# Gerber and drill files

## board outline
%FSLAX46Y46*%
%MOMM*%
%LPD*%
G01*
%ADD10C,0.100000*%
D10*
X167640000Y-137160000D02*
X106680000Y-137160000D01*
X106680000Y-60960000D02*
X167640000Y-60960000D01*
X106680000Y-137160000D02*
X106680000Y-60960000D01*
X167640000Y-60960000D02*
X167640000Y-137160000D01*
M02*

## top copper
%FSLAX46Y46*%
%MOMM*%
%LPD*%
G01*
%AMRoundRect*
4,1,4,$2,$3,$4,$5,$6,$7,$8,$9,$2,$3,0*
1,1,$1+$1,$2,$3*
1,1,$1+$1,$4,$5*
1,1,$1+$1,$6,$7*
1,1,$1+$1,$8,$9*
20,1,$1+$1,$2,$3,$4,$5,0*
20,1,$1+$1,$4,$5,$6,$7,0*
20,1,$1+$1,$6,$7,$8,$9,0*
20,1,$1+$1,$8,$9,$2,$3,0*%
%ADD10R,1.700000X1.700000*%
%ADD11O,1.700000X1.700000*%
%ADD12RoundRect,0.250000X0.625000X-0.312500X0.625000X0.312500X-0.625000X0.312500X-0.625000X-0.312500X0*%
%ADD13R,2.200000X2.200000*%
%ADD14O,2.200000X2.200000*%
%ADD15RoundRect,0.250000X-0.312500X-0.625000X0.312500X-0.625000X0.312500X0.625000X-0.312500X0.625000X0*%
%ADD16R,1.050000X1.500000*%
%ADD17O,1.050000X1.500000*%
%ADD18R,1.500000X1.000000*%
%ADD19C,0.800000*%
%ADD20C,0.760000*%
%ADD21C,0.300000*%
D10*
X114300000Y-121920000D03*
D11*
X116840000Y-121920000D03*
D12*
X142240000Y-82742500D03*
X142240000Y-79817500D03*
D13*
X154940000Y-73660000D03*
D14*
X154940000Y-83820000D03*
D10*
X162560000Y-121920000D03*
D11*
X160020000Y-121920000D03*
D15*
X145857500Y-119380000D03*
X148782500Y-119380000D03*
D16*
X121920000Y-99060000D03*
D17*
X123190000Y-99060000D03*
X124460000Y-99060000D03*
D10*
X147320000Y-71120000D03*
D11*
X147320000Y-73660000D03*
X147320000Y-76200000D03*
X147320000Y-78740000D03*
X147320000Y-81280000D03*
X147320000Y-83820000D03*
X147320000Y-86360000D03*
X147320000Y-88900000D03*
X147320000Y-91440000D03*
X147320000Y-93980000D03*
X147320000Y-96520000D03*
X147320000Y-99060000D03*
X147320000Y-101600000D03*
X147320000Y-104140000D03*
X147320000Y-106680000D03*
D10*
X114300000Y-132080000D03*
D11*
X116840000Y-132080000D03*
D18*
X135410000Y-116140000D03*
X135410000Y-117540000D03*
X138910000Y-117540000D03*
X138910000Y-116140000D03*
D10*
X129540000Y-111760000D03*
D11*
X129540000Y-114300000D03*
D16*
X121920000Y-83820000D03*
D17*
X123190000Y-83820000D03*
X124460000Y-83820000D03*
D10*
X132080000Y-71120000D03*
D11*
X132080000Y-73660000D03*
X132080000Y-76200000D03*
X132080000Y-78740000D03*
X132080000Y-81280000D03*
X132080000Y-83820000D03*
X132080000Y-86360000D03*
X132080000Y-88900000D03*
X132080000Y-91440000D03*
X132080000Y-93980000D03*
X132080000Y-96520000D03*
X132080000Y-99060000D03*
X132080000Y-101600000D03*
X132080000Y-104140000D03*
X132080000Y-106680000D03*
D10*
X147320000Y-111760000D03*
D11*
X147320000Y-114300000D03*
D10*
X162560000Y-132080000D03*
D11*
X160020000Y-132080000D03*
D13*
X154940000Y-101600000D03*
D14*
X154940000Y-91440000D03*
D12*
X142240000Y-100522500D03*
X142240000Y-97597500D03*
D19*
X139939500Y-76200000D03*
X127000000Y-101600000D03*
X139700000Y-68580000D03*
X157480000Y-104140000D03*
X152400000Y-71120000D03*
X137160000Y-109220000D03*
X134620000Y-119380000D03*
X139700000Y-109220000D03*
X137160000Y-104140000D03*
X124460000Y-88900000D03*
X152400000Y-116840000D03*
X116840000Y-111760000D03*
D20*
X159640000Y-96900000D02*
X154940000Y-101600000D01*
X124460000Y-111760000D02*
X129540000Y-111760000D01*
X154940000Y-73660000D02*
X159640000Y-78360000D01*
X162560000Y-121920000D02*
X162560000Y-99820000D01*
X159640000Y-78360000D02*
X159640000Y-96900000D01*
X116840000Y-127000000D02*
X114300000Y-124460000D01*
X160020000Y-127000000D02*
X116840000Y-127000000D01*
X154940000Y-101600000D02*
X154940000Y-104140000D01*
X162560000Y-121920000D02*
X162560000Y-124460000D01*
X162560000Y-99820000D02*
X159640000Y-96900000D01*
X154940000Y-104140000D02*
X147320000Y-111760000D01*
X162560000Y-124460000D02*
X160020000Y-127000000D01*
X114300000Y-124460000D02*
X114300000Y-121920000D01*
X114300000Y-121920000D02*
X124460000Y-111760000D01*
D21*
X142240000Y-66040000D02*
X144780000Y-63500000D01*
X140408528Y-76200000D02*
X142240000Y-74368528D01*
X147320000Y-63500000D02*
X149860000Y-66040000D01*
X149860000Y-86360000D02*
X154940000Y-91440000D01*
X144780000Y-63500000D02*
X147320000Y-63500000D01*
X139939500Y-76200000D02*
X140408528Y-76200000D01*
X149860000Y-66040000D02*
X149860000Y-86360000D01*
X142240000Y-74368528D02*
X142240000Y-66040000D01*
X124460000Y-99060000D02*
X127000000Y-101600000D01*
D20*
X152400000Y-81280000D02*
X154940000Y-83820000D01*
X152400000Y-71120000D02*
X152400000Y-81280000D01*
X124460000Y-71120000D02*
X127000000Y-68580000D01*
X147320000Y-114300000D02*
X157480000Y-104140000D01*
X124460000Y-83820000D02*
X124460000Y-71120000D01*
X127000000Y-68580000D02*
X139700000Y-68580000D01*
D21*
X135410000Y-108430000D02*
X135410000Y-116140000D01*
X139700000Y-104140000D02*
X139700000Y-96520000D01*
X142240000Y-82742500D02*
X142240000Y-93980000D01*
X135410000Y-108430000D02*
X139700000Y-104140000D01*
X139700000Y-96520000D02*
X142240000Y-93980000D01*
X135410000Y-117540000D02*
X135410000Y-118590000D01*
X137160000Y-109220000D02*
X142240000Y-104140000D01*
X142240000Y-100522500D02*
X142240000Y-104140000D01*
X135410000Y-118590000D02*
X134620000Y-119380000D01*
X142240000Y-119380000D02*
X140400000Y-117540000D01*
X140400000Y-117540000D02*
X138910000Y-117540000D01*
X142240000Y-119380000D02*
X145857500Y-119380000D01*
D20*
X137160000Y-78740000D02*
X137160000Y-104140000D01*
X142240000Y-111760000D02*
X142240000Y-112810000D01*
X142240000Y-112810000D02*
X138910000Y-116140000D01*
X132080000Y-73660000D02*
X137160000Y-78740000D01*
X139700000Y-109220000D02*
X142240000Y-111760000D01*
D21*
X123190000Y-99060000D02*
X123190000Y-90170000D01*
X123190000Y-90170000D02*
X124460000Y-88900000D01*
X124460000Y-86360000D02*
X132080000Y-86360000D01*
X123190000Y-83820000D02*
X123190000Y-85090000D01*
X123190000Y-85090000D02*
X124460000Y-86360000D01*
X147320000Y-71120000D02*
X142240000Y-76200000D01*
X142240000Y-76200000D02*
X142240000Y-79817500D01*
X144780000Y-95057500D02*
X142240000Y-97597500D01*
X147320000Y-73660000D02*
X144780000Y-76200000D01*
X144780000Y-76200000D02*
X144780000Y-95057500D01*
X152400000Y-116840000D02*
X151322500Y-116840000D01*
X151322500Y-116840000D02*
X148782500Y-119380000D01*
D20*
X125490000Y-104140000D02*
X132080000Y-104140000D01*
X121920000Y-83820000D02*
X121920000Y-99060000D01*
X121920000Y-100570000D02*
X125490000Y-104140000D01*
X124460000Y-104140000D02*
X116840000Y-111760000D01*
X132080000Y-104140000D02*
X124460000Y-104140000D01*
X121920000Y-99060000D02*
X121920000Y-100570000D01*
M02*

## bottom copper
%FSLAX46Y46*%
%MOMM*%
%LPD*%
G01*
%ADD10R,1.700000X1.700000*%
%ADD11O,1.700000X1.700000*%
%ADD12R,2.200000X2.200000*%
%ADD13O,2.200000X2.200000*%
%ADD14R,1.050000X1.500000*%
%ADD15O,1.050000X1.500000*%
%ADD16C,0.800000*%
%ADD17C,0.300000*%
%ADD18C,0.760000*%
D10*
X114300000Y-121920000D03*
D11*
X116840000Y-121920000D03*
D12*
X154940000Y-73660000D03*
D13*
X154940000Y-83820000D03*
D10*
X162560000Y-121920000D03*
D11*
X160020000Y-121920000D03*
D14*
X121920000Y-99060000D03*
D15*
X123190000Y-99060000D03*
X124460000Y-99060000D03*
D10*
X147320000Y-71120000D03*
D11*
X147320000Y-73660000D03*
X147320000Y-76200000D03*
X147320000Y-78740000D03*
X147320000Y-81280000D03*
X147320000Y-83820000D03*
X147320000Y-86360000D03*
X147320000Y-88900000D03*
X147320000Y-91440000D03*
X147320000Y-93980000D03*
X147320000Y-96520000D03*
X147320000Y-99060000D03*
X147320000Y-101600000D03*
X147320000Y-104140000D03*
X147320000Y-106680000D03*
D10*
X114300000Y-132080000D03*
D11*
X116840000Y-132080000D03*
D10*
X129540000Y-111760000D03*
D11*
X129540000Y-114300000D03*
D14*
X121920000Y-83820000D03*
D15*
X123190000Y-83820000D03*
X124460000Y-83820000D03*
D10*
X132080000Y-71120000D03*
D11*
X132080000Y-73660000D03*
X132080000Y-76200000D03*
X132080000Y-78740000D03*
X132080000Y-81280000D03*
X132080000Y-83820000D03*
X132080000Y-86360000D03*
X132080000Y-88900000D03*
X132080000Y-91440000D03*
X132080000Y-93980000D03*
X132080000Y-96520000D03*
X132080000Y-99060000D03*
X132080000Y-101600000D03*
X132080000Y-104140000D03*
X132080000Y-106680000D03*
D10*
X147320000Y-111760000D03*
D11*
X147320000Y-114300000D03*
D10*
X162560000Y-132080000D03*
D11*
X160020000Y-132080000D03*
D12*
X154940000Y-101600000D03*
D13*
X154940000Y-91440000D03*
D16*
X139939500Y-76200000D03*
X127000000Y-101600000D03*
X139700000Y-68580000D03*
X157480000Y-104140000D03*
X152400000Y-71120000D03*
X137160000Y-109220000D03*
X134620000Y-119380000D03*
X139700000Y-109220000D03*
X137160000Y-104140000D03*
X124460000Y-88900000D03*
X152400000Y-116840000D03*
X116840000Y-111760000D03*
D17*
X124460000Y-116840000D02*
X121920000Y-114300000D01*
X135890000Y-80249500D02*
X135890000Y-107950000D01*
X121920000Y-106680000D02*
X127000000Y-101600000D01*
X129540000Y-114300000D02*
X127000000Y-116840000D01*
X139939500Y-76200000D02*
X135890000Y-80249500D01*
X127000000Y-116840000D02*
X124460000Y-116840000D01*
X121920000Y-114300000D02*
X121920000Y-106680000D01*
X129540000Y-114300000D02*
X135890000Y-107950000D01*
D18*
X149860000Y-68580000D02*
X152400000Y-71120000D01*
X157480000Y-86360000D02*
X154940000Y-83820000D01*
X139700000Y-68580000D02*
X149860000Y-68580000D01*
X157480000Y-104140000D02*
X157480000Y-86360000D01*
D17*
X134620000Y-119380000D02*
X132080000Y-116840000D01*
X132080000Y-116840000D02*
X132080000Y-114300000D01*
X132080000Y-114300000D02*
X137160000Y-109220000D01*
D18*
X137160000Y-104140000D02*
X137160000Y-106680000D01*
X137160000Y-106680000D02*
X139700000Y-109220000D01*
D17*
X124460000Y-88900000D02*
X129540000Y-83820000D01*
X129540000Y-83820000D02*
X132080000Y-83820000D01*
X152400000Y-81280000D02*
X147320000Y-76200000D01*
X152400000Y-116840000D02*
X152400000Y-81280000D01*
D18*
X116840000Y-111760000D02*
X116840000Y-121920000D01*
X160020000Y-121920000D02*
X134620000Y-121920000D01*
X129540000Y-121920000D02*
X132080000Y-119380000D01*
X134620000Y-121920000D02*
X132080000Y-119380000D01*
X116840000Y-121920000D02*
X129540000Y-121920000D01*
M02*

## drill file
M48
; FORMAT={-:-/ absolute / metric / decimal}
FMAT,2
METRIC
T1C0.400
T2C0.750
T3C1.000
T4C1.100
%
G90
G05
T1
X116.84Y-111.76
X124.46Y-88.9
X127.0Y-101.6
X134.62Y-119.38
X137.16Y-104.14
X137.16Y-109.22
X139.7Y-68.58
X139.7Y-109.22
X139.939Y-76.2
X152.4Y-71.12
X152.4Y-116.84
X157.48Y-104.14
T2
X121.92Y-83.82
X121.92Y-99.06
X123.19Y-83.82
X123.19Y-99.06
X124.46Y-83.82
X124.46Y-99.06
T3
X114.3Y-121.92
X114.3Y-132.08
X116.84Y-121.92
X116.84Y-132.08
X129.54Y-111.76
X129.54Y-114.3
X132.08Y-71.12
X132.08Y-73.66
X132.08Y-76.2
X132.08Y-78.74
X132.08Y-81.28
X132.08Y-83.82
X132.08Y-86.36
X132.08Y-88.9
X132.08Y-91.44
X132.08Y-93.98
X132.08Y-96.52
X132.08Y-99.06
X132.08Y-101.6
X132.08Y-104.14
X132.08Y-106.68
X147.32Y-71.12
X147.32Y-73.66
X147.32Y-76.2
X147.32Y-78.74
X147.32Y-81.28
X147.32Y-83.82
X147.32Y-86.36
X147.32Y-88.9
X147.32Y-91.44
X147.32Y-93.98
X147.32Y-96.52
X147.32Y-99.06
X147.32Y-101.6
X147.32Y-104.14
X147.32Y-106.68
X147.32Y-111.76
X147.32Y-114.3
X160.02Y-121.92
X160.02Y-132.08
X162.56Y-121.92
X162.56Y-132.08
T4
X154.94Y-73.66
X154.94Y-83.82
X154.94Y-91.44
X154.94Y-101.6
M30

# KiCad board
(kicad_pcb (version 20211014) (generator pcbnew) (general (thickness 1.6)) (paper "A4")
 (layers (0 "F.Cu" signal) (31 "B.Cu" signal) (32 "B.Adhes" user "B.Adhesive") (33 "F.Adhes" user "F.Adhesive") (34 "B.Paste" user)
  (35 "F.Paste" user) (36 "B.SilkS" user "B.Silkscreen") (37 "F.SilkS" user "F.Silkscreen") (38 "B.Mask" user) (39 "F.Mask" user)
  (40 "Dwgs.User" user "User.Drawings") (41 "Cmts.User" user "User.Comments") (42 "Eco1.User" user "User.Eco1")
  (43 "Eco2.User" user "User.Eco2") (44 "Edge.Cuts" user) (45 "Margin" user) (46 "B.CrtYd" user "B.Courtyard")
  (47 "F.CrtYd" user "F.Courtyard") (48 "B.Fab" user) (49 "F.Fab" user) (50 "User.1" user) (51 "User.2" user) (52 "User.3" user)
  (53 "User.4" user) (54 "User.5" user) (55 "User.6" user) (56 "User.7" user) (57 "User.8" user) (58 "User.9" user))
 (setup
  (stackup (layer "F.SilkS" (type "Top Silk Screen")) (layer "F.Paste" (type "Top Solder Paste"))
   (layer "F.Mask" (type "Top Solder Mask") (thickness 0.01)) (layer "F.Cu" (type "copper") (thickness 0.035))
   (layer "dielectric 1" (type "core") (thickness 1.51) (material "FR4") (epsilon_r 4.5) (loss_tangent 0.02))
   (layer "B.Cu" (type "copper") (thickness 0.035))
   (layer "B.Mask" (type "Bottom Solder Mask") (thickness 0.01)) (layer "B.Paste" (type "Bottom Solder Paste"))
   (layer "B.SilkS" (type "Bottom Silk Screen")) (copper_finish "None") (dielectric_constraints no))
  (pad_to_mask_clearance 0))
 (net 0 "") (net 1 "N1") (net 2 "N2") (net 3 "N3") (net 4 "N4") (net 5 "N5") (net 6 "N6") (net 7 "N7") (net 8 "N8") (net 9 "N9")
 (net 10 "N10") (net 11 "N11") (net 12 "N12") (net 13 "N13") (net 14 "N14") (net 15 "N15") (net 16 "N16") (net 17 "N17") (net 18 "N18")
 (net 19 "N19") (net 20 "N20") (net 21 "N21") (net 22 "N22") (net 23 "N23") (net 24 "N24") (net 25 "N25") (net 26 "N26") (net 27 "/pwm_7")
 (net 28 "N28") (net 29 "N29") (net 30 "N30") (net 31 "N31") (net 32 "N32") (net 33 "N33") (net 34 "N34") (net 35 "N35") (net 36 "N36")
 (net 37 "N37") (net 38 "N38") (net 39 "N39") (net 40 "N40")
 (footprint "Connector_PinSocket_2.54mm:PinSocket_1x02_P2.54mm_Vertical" (layer "F.Cu") (at 114.3 121.92 90)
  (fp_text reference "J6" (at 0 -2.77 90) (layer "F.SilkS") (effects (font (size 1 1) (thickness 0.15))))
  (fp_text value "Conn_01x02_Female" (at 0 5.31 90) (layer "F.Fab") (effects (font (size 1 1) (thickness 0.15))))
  (pad "1" thru_hole rect (at 0 0 90) (size 1.7 1.7) (drill 1) (layers *.Cu *.Mask) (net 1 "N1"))
  (pad "2" thru_hole oval (at 0 2.54 90) (size 1.7 1.7) (drill 1) (layers *.Cu *.Mask) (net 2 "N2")))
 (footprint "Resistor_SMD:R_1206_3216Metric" (layer "F.Cu") (at 142.24 81.28 90)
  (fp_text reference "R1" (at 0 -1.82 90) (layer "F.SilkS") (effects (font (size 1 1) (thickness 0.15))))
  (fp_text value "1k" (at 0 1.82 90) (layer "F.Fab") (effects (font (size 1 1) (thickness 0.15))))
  (pad "1" smd roundrect (at -1.4625 0 90) (size 1.125 1.75) (layers "F.Cu" "F.Paste" "F.Mask") (roundrect_rratio 0.222222) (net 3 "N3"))
  (pad "2" smd roundrect (at 1.4625 0 90) (size 1.125 1.75) (layers "F.Cu" "F.Paste" "F.Mask") (roundrect_rratio 0.222222) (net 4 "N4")))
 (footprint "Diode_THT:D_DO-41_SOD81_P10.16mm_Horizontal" (layer "F.Cu") (at 154.94 73.66 -90)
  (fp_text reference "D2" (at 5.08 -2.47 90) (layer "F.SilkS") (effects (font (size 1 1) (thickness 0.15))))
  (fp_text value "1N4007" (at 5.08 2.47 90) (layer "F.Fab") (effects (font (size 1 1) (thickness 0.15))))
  (pad "1" thru_hole rect (at 0 0 270) (size 2.2 2.2) (drill 1.1) (layers *.Cu *.Mask) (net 1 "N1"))
  (pad "2" thru_hole oval (at 10.16 0 270) (size 2.2 2.2) (drill 1.1) (layers *.Cu *.Mask) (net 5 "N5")))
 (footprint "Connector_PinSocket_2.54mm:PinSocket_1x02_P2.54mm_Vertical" (layer "F.Cu") (at 162.56 121.92 -90)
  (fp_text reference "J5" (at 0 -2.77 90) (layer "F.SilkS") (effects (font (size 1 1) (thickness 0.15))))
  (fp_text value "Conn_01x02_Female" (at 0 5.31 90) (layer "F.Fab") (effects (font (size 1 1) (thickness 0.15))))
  (pad "1" thru_hole rect (at 0 0 270) (size 1.7 1.7) (drill 1) (layers *.Cu *.Mask) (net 1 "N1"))
  (pad "2" thru_hole oval (at 0 2.54 270) (size 1.7 1.7) (drill 1) (layers *.Cu *.Mask) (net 2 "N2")))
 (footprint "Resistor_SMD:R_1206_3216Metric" (layer "F.Cu") (at 147.32 119.38)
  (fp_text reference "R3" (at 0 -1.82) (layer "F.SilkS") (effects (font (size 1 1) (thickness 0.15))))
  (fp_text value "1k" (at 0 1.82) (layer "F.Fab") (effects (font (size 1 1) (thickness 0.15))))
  (pad "1" smd roundrect (at -1.4625 0) (size 1.125 1.75) (layers "F.Cu" "F.Paste" "F.Mask") (roundrect_rratio 0.222222) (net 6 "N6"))
  (pad "2" smd roundrect (at 1.4625 0) (size 1.125 1.75) (layers "F.Cu" "F.Paste" "F.Mask") (roundrect_rratio 0.222222) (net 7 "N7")))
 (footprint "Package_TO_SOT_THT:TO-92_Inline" (layer "F.Cu") (at 121.92 99.06)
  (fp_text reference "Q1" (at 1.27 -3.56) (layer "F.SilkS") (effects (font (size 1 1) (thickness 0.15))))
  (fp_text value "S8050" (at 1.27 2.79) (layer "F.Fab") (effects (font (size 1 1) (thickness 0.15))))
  (pad "1" thru_hole rect (at 0 0) (size 1.05 1.5) (drill 0.75) (layers *.Cu *.Mask) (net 2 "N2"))
  (pad "2" thru_hole oval (at 1.27 0) (size 1.05 1.5) (drill 0.75) (layers *.Cu *.Mask) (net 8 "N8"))
  (pad "3" thru_hole oval (at 2.54 0) (size 1.05 1.5) (drill 0.75) (layers *.Cu *.Mask) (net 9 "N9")))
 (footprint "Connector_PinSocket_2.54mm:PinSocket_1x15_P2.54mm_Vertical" (layer "F.Cu") (at 147.32 71.12)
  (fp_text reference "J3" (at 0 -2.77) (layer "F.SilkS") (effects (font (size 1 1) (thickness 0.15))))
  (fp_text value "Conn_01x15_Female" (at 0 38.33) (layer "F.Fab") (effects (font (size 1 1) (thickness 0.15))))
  (pad "1" thru_hole rect (at 0 0) (size 1.7 1.7) (drill 1) (layers *.Cu *.Mask) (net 4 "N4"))
  (pad "2" thru_hole oval (at 0 2.54) (size 1.7 1.7) (drill 1) (layers *.Cu *.Mask) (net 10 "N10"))
  (pad "3" thru_hole oval (at 0 5.08) (size 1.7 1.7) (drill 1) (layers *.Cu *.Mask) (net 7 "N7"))
  (pad "4" thru_hole oval (at 0 7.62) (size 1.7 1.7) (drill 1) (layers *.Cu *.Mask) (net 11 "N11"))
  (pad "5" thru_hole oval (at 0 10.16) (size 1.7 1.7) (drill 1) (layers *.Cu *.Mask) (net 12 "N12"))
  (pad "6" thru_hole oval (at 0 12.7) (size 1.7 1.7) (drill 1) (layers *.Cu *.Mask) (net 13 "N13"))
  (pad "7" thru_hole oval (at 0 15.24) (size 1.7 1.7) (drill 1) (layers *.Cu *.Mask) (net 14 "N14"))
  (pad "8" thru_hole oval (at 0 17.78) (size 1.7 1.7) (drill 1) (layers *.Cu *.Mask) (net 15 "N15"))
  (pad "9" thru_hole oval (at 0 20.32) (size 1.7 1.7) (drill 1) (layers *.Cu *.Mask) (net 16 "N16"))
  (pad "10" thru_hole oval (at 0 22.86) (size 1.7 1.7) (drill 1) (layers *.Cu *.Mask) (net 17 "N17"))
  (pad "11" thru_hole oval (at 0 25.4) (size 1.7 1.7) (drill 1) (layers *.Cu *.Mask) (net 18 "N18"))
  (pad "12" thru_hole oval (at 0 27.94) (size 1.7 1.7) (drill 1) (layers *.Cu *.Mask) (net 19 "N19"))
  (pad "13" thru_hole oval (at 0 30.48) (size 1.7 1.7) (drill 1) (layers *.Cu *.Mask) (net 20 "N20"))
  (pad "14" thru_hole oval (at 0 33.02) (size 1.7 1.7) (drill 1) (layers *.Cu *.Mask) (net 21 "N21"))
  (pad "15" thru_hole oval (at 0 35.56) (size 1.7 1.7) (drill 1) (layers *.Cu *.Mask) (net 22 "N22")))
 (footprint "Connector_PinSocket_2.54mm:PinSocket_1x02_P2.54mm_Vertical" (layer "F.Cu") (at 114.3 132.08 90)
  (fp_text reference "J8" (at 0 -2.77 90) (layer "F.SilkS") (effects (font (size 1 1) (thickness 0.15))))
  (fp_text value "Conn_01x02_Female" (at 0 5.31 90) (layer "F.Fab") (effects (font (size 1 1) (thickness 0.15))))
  (pad "1" thru_hole rect (at 0 0 90) (size 1.7 1.7) (drill 1) (layers *.Cu *.Mask) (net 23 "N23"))
  (pad "2" thru_hole oval (at 0 2.54 90) (size 1.7 1.7) (drill 1) (layers *.Cu *.Mask) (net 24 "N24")))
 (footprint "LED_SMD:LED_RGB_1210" (layer "F.Cu") (at 137.16 116.84)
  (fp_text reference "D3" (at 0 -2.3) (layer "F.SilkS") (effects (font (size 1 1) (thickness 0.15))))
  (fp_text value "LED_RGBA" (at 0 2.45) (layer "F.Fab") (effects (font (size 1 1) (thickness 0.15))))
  (pad "1" smd rect (at -1.75 -0.7 180) (size 1.5 1) (layers "F.Cu" "F.Paste" "F.Mask") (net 3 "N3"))
  (pad "2" smd rect (at -1.75 0.7 180) (size 1.5 1) (layers "F.Cu" "F.Paste" "F.Mask") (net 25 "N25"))
  (pad "3" smd rect (at 1.75 0.7 180) (size 1.5 1) (layers "F.Cu" "F.Paste" "F.Mask") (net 6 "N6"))
  (pad "4" smd rect (at 1.75 -0.7 180) (size 1.5 1) (layers "F.Cu" "F.Paste" "F.Mask") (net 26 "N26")))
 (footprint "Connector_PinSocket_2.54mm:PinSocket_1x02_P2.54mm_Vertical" (layer "F.Cu") (at 129.54 111.76)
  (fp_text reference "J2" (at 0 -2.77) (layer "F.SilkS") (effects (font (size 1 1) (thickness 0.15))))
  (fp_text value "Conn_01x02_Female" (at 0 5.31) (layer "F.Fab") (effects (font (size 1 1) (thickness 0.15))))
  (pad "1" thru_hole rect (at 0 0) (size 1.7 1.7) (drill 1) (layers *.Cu *.Mask) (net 1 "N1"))
  (pad "2" thru_hole oval (at 0 2.54) (size 1.7 1.7) (drill 1) (layers *.Cu *.Mask) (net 9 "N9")))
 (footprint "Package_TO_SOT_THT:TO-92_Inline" (layer "F.Cu") (at 121.92 83.82)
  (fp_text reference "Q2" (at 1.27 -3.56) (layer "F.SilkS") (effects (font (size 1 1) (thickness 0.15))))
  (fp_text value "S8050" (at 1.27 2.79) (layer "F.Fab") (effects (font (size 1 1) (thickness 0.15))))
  (pad "1" thru_hole rect (at 0 0) (size 1.05 1.5) (drill 0.75) (layers *.Cu *.Mask) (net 2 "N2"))
  (pad "2" thru_hole oval (at 1.27 0) (size 1.05 1.5) (drill 0.75) (layers *.Cu *.Mask) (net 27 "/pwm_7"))
  (pad "3" thru_hole oval (at 2.54 0) (size 1.05 1.5) (drill 0.75) (layers *.Cu *.Mask) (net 5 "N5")))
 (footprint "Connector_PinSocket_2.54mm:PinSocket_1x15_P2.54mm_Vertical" (layer "F.Cu") (at 132.08 71.12)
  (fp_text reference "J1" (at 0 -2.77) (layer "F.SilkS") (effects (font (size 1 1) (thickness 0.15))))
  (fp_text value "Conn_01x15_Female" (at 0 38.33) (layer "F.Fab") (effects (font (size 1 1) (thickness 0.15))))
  (pad "1" thru_hole rect (at 0 0) (size 1.7 1.7) (drill 1) (layers *.Cu *.Mask) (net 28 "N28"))
  (pad "2" thru_hole oval (at 0 2.54) (size 1.7 1.7) (drill 1) (layers *.Cu *.Mask) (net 26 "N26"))
  (pad "3" thru_hole oval (at 0 5.08) (size 1.7 1.7) (drill 1) (layers *.Cu *.Mask) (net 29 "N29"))
  (pad "4" thru_hole oval (at 0 7.62) (size 1.7 1.7) (drill 1) (layers *.Cu *.Mask) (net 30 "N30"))
  (pad "5" thru_hole oval (at 0 10.16) (size 1.7 1.7) (drill 1) (layers *.Cu *.Mask) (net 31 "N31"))
  (pad "6" thru_hole oval (at 0 12.7) (size 1.7 1.7) (drill 1) (layers *.Cu *.Mask) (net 8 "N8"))
  (pad "7" thru_hole oval (at 0 15.24) (size 1.7 1.7) (drill 1) (layers *.Cu *.Mask) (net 27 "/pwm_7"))
  (pad "8" thru_hole oval (at 0 17.78) (size 1.7 1.7) (drill 1) (layers *.Cu *.Mask) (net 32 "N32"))
  (pad "9" thru_hole oval (at 0 20.32) (size 1.7 1.7) (drill 1) (layers *.Cu *.Mask) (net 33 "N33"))
  (pad "10" thru_hole oval (at 0 22.86) (size 1.7 1.7) (drill 1) (layers *.Cu *.Mask) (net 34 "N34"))
  (pad "11" thru_hole oval (at 0 25.4) (size 1.7 1.7) (drill 1) (layers *.Cu *.Mask) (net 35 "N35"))
  (pad "12" thru_hole oval (at 0 27.94) (size 1.7 1.7) (drill 1) (layers *.Cu *.Mask) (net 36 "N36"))
  (pad "13" thru_hole oval (at 0 30.48) (size 1.7 1.7) (drill 1) (layers *.Cu *.Mask) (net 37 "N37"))
  (pad "14" thru_hole oval (at 0 33.02) (size 1.7 1.7) (drill 1) (layers *.Cu *.Mask) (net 2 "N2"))
  (pad "15" thru_hole oval (at 0 35.56) (size 1.7 1.7) (drill 1) (layers *.Cu *.Mask) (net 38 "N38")))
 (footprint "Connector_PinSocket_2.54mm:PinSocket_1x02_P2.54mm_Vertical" (layer "F.Cu") (at 147.32 111.76)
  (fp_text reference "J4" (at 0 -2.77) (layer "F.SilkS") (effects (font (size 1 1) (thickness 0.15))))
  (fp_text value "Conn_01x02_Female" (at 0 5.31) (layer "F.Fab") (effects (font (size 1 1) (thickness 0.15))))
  (pad "1" thru_hole rect (at 0 0) (size 1.7 1.7) (drill 1) (layers *.Cu *.Mask) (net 1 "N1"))
  (pad "2" thru_hole oval (at 0 2.54) (size 1.7 1.7) (drill 1) (layers *.Cu *.Mask) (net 5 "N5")))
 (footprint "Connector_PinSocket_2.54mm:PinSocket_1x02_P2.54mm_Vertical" (layer "F.Cu") (at 162.56 132.08 -90)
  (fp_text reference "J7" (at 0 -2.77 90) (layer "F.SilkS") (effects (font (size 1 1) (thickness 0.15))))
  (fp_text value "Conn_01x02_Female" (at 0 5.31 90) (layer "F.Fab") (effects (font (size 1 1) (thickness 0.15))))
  (pad "1" thru_hole rect (at 0 0 270) (size 1.7 1.7) (drill 1) (layers *.Cu *.Mask) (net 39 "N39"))
  (pad "2" thru_hole oval (at 0 2.54 270) (size 1.7 1.7) (drill 1) (layers *.Cu *.Mask) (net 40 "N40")))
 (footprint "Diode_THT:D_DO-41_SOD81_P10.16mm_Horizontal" (layer "F.Cu") (at 154.94 101.6 90)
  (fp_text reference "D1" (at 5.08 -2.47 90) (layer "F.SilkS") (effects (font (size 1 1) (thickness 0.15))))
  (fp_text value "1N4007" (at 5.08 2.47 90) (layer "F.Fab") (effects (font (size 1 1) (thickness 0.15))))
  (pad "1" thru_hole rect (at 0 0 90) (size 2.2 2.2) (drill 1.1) (layers *.Cu *.Mask) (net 1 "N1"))
  (pad "2" thru_hole oval (at 10.16 0 90) (size 2.2 2.2) (drill 1.1) (layers *.Cu *.Mask) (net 9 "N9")))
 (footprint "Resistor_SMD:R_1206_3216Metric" (layer "F.Cu") (at 142.24 99.06 90)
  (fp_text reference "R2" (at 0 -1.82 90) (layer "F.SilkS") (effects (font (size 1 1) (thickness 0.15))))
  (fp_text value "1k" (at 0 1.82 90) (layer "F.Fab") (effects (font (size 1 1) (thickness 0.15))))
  (pad "1" smd roundrect (at -1.4625 0 90) (size 1.125 1.75) (layers "F.Cu" "F.Paste" "F.Mask") (roundrect_rratio 0.222222) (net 25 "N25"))
  (pad "2" smd roundrect (at 1.4625 0 90) (size 1.125 1.75) (layers "F.Cu" "F.Paste" "F.Mask") (roundrect_rratio 0.222222) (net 10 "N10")))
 (gr_line (start 167.64 137.16) (end 106.68 137.16) (layer "Edge.Cuts") (width 0.1))
 (gr_line (start 106.68 60.96) (end 167.64 60.96) (layer "Edge.Cuts") (width 0.1))
 (gr_line (start 106.68 137.16) (end 106.68 60.96) (layer "Edge.Cuts") (width 0.1))
 (gr_line (start 167.64 60.96) (end 167.64 137.16) (layer "Edge.Cuts") (width 0.1))
 (segment (start 159.64 96.9) (end 154.94 101.6) (width 0.76) (layer "F.Cu") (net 1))
 (segment (start 124.46 111.76) (end 129.54 111.76) (width 0.76) (layer "F.Cu") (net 1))
 (segment (start 154.94 73.66) (end 159.64 78.36) (width 0.76) (layer "F.Cu") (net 1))
 (segment (start 162.56 121.92) (end 162.56 99.82) (width 0.76) (layer "F.Cu") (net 1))
 (segment (start 159.64 78.36) (end 159.64 96.9) (width 0.76) (layer "F.Cu") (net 1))
 (segment (start 116.84 127) (end 114.3 124.46) (width 0.76) (layer "F.Cu") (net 1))
 (segment (start 160.02 127) (end 116.84 127) (width 0.76) (layer "F.Cu") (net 1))
 (segment (start 154.94 101.6) (end 154.94 104.14) (width 0.76) (layer "F.Cu") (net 1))
 (segment (start 162.56 121.92) (end 162.56 124.46) (width 0.76) (layer "F.Cu") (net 1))
 (segment (start 162.56 99.82) (end 159.64 96.9) (width 0.76) (layer "F.Cu") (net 1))
 (segment (start 154.94 104.14) (end 147.32 111.76) (width 0.76) (layer "F.Cu") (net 1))
 (segment (start 162.56 124.46) (end 160.02 127) (width 0.76) (layer "F.Cu") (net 1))
 (segment (start 114.3 124.46) (end 114.3 121.92) (width 0.76) (layer "F.Cu") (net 1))
 (segment (start 114.3 121.92) (end 124.46 111.76) (width 0.76) (layer "F.Cu") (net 1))
 (segment (start 142.24 66.04) (end 144.78 63.5) (width 0.3) (layer "F.Cu") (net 9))
 (segment (start 140.408528 76.2) (end 142.24 74.368528) (width 0.3) (layer "F.Cu") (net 9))
 (segment (start 147.32 63.5) (end 149.86 66.04) (width 0.3) (layer "F.Cu") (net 9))
 (segment (start 149.86 86.36) (end 154.94 91.44) (width 0.3) (layer "F.Cu") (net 9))
 (segment (start 144.78 63.5) (end 147.32 63.5) (width 0.3) (layer "F.Cu") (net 9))
 (segment (start 139.9395 76.2) (end 140.408528 76.2) (width 0.3) (layer "F.Cu") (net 9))
 (segment (start 149.86 66.04) (end 149.86 86.36) (width 0.3) (layer "F.Cu") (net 9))
 (segment (start 142.24 74.368528) (end 142.24 66.04) (width 0.3) (layer "F.Cu") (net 9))
 (segment (start 124.46 99.06) (end 127 101.6) (width 0.3) (layer "F.Cu") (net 9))
 (via (at 139.9395 76.2) (size 0.8) (drill 0.4) (layers "F.Cu" "B.Cu") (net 9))
 (via (at 127 101.6) (size 0.8) (drill 0.4) (layers "F.Cu" "B.Cu") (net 9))
 (segment (start 124.46 116.84) (end 121.92 114.3) (width 0.3) (layer "B.Cu") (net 9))
 (segment (start 135.89 80.2495) (end 135.89 107.95) (width 0.3) (layer "B.Cu") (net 9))
 (segment (start 121.92 106.68) (end 127 101.6) (width 0.3) (layer "B.Cu") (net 9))
 (segment (start 129.54 114.3) (end 127 116.84) (width 0.3) (layer "B.Cu") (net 9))
 (segment (start 139.9395 76.2) (end 135.89 80.2495) (width 0.3) (layer "B.Cu") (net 9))
 (segment (start 127 116.84) (end 124.46 116.84) (width 0.3) (layer "B.Cu") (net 9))
 (segment (start 121.92 114.3) (end 121.92 106.68) (width 0.3) (layer "B.Cu") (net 9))
 (segment (start 129.54 114.3) (end 135.89 107.95) (width 0.3) (layer "B.Cu") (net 9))
 (segment (start 152.4 81.28) (end 154.94 83.82) (width 0.76) (layer "F.Cu") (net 5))
 (segment (start 152.4 71.12) (end 152.4 81.28) (width 0.76) (layer "F.Cu") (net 5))
 (segment (start 124.46 71.12) (end 127 68.58) (width 0.76) (layer "F.Cu") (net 5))
 (segment (start 147.32 114.3) (end 157.48 104.14) (width 0.76) (layer "F.Cu") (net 5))
 (segment (start 124.46 83.82) (end 124.46 71.12) (width 0.76) (layer "F.Cu") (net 5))
 (segment (start 127 68.58) (end 139.7 68.58) (width 0.76) (layer "F.Cu") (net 5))
 (via (at 139.7 68.58) (size 0.8) (drill 0.4) (layers "F.Cu" "B.Cu") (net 5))
 (via (at 157.48 104.14) (size 0.8) (drill 0.4) (layers "F.Cu" "B.Cu") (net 5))
 (via (at 152.4 71.12) (size 0.8) (drill 0.4) (layers "F.Cu" "B.Cu") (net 5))
 (segment (start 149.86 68.58) (end 152.4 71.12) (width 0.76) (layer "B.Cu") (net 5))
 (segment (start 157.48 86.36) (end 154.94 83.82) (width 0.76) (layer "B.Cu") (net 5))
 (segment (start 139.7 68.58) (end 149.86 68.58) (width 0.76) (layer "B.Cu") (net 5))
 (segment (start 157.48 104.14) (end 157.48 86.36) (width 0.76) (layer "B.Cu") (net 5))
 (segment (start 135.41 108.43) (end 135.41 116.14) (width 0.3) (layer "F.Cu") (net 3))
 (segment (start 139.7 104.14) (end 139.7 96.52) (width 0.3) (layer "F.Cu") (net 3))
 (segment (start 142.24 82.7425) (end 142.24 93.98) (width 0.3) (layer "F.Cu") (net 3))
 (segment (start 135.41 108.43) (end 139.7 104.14) (width 0.3) (layer "F.Cu") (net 3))
 (segment (start 139.7 96.52) (end 142.24 93.98) (width 0.3) (layer "F.Cu") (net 3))
 (segment (start 135.41 117.54) (end 135.41 118.59) (width 0.3) (layer "F.Cu") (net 25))
 (segment (start 137.16 109.22) (end 142.24 104.14) (width 0.3) (layer "F.Cu") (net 25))
 (segment (start 142.24 100.5225) (end 142.24 104.14) (width 0.3) (layer "F.Cu") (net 25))
 (segment (start 135.41 118.59) (end 134.62 119.38) (width 0.3) (layer "F.Cu") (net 25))
 (via (at 137.16 109.22) (size 0.8) (drill 0.4) (layers "F.Cu" "B.Cu") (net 25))
 (via (at 134.62 119.38) (size 0.8) (drill 0.4) (layers "F.Cu" "B.Cu") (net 25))
 (segment (start 134.62 119.38) (end 132.08 116.84) (width 0.3) (layer "B.Cu") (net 25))
 (segment (start 132.08 116.84) (end 132.08 114.3) (width 0.3) (layer "B.Cu") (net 25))
 (segment (start 132.08 114.3) (end 137.16 109.22) (width 0.3) (layer "B.Cu") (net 25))
 (segment (start 142.24 119.38) (end 140.4 117.54) (width 0.3) (layer "F.Cu") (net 6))
 (segment (start 140.4 117.54) (end 138.91 117.54) (width 0.3) (layer "F.Cu") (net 6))
 (segment (start 142.24 119.38) (end 145.8575 119.38) (width 0.3) (layer "F.Cu") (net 6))
 (segment (start 137.16 78.74) (end 137.16 104.14) (width 0.76) (layer "F.Cu") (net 26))
 (segment (start 142.24 111.76) (end 142.24 112.81) (width 0.76) (layer "F.Cu") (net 26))
 (segment (start 142.24 112.81) (end 138.91 116.14) (width 0.76) (layer "F.Cu") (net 26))
 (segment (start 132.08 73.66) (end 137.16 78.74) (width 0.76) (layer "F.Cu") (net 26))
 (segment (start 139.7 109.22) (end 142.24 111.76) (width 0.76) (layer "F.Cu") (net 26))
 (via (at 139.7 109.22) (size 0.8) (drill 0.4) (layers "F.Cu" "B.Cu") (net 26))
 (via (at 137.16 104.14) (size 0.8) (drill 0.4) (layers "F.Cu" "B.Cu") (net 26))
 (segment (start 137.16 104.14) (end 137.16 106.68) (width 0.76) (layer "B.Cu") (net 26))
 (segment (start 137.16 106.68) (end 139.7 109.22) (width 0.76) (layer "B.Cu") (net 26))
 (segment (start 123.19 99.06) (end 123.19 90.17) (width 0.3) (layer "F.Cu") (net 8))
 (segment (start 123.19 90.17) (end 124.46 88.9) (width 0.3) (layer "F.Cu") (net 8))
 (via (at 124.46 88.9) (size 0.8) (drill 0.4) (layers "F.Cu" "B.Cu") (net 8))
 (segment (start 124.46 88.9) (end 129.54 83.82) (width 0.3) (layer "B.Cu") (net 8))
 (segment (start 129.54 83.82) (end 132.08 83.82) (width 0.3) (layer "B.Cu") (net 8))
 (segment (start 124.46 86.36) (end 132.08 86.36) (width 0.3) (layer "F.Cu") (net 27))
 (segment (start 123.19 83.82) (end 123.19 85.09) (width 0.3) (layer "F.Cu") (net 27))
 (segment (start 123.19 85.09) (end 124.46 86.36) (width 0.3) (layer "F.Cu") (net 27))
 (segment (start 147.32 71.12) (end 142.24 76.2) (width 0.3) (layer "F.Cu") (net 4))
 (segment (start 142.24 76.2) (end 142.24 79.8175) (width 0.3) (layer "F.Cu") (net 4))
 (segment (start 144.78 95.0575) (end 142.24 97.5975) (width 0.3) (layer "F.Cu") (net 10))
 (segment (start 147.32 73.66) (end 144.78 76.2) (width 0.3) (layer "F.Cu") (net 10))
 (segment (start 144.78 76.2) (end 144.78 95.0575) (width 0.3) (layer "F.Cu") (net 10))
 (segment (start 152.4 116.84) (end 151.3225 116.84) (width 0.3) (layer "F.Cu") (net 7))
 (segment (start 151.3225 116.84) (end 148.7825 119.38) (width 0.3) (layer "F.Cu") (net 7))
 (via (at 152.4 116.84) (size 0.8) (drill 0.4) (layers "F.Cu" "B.Cu") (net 7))
 (segment (start 152.4 81.28) (end 147.32 76.2) (width 0.3) (layer "B.Cu") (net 7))
 (segment (start 152.4 116.84) (end 152.4 81.28) (width 0.3) (layer "B.Cu") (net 7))
 (segment (start 125.49 104.14) (end 132.08 104.14) (width 0.76) (layer "F.Cu") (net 2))
 (segment (start 121.92 83.82) (end 121.92 99.06) (width 0.76) (layer "F.Cu") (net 2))
 (segment (start 121.92 100.57) (end 125.49 104.14) (width 0.76) (layer "F.Cu") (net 2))
 (segment (start 124.46 104.14) (end 116.84 111.76) (width 0.76) (layer "F.Cu") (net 2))
 (segment (start 132.08 104.14) (end 124.46 104.14) (width 0.76) (layer "F.Cu") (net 2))
 (segment (start 121.92 99.06) (end 121.92 100.57) (width 0.76) (layer "F.Cu") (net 2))
 (via (at 116.84 111.76) (size 0.8) (drill 0.4) (layers "F.Cu" "B.Cu") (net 2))
 (segment (start 116.84 111.76) (end 116.84 121.92) (width 0.76) (layer "B.Cu") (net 2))
 (segment (start 160.02 121.92) (end 134.62 121.92) (width 0.76) (layer "B.Cu") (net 2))
 (segment (start 129.54 121.92) (end 132.08 119.38) (width 0.76) (layer "B.Cu") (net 2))
 (segment (start 134.62 121.92) (end 132.08 119.38) (width 0.76) (layer "B.Cu") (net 2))
 (segment (start 116.84 121.92) (end 129.54 121.92) (width 0.76) (layer "B.Cu") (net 2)))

